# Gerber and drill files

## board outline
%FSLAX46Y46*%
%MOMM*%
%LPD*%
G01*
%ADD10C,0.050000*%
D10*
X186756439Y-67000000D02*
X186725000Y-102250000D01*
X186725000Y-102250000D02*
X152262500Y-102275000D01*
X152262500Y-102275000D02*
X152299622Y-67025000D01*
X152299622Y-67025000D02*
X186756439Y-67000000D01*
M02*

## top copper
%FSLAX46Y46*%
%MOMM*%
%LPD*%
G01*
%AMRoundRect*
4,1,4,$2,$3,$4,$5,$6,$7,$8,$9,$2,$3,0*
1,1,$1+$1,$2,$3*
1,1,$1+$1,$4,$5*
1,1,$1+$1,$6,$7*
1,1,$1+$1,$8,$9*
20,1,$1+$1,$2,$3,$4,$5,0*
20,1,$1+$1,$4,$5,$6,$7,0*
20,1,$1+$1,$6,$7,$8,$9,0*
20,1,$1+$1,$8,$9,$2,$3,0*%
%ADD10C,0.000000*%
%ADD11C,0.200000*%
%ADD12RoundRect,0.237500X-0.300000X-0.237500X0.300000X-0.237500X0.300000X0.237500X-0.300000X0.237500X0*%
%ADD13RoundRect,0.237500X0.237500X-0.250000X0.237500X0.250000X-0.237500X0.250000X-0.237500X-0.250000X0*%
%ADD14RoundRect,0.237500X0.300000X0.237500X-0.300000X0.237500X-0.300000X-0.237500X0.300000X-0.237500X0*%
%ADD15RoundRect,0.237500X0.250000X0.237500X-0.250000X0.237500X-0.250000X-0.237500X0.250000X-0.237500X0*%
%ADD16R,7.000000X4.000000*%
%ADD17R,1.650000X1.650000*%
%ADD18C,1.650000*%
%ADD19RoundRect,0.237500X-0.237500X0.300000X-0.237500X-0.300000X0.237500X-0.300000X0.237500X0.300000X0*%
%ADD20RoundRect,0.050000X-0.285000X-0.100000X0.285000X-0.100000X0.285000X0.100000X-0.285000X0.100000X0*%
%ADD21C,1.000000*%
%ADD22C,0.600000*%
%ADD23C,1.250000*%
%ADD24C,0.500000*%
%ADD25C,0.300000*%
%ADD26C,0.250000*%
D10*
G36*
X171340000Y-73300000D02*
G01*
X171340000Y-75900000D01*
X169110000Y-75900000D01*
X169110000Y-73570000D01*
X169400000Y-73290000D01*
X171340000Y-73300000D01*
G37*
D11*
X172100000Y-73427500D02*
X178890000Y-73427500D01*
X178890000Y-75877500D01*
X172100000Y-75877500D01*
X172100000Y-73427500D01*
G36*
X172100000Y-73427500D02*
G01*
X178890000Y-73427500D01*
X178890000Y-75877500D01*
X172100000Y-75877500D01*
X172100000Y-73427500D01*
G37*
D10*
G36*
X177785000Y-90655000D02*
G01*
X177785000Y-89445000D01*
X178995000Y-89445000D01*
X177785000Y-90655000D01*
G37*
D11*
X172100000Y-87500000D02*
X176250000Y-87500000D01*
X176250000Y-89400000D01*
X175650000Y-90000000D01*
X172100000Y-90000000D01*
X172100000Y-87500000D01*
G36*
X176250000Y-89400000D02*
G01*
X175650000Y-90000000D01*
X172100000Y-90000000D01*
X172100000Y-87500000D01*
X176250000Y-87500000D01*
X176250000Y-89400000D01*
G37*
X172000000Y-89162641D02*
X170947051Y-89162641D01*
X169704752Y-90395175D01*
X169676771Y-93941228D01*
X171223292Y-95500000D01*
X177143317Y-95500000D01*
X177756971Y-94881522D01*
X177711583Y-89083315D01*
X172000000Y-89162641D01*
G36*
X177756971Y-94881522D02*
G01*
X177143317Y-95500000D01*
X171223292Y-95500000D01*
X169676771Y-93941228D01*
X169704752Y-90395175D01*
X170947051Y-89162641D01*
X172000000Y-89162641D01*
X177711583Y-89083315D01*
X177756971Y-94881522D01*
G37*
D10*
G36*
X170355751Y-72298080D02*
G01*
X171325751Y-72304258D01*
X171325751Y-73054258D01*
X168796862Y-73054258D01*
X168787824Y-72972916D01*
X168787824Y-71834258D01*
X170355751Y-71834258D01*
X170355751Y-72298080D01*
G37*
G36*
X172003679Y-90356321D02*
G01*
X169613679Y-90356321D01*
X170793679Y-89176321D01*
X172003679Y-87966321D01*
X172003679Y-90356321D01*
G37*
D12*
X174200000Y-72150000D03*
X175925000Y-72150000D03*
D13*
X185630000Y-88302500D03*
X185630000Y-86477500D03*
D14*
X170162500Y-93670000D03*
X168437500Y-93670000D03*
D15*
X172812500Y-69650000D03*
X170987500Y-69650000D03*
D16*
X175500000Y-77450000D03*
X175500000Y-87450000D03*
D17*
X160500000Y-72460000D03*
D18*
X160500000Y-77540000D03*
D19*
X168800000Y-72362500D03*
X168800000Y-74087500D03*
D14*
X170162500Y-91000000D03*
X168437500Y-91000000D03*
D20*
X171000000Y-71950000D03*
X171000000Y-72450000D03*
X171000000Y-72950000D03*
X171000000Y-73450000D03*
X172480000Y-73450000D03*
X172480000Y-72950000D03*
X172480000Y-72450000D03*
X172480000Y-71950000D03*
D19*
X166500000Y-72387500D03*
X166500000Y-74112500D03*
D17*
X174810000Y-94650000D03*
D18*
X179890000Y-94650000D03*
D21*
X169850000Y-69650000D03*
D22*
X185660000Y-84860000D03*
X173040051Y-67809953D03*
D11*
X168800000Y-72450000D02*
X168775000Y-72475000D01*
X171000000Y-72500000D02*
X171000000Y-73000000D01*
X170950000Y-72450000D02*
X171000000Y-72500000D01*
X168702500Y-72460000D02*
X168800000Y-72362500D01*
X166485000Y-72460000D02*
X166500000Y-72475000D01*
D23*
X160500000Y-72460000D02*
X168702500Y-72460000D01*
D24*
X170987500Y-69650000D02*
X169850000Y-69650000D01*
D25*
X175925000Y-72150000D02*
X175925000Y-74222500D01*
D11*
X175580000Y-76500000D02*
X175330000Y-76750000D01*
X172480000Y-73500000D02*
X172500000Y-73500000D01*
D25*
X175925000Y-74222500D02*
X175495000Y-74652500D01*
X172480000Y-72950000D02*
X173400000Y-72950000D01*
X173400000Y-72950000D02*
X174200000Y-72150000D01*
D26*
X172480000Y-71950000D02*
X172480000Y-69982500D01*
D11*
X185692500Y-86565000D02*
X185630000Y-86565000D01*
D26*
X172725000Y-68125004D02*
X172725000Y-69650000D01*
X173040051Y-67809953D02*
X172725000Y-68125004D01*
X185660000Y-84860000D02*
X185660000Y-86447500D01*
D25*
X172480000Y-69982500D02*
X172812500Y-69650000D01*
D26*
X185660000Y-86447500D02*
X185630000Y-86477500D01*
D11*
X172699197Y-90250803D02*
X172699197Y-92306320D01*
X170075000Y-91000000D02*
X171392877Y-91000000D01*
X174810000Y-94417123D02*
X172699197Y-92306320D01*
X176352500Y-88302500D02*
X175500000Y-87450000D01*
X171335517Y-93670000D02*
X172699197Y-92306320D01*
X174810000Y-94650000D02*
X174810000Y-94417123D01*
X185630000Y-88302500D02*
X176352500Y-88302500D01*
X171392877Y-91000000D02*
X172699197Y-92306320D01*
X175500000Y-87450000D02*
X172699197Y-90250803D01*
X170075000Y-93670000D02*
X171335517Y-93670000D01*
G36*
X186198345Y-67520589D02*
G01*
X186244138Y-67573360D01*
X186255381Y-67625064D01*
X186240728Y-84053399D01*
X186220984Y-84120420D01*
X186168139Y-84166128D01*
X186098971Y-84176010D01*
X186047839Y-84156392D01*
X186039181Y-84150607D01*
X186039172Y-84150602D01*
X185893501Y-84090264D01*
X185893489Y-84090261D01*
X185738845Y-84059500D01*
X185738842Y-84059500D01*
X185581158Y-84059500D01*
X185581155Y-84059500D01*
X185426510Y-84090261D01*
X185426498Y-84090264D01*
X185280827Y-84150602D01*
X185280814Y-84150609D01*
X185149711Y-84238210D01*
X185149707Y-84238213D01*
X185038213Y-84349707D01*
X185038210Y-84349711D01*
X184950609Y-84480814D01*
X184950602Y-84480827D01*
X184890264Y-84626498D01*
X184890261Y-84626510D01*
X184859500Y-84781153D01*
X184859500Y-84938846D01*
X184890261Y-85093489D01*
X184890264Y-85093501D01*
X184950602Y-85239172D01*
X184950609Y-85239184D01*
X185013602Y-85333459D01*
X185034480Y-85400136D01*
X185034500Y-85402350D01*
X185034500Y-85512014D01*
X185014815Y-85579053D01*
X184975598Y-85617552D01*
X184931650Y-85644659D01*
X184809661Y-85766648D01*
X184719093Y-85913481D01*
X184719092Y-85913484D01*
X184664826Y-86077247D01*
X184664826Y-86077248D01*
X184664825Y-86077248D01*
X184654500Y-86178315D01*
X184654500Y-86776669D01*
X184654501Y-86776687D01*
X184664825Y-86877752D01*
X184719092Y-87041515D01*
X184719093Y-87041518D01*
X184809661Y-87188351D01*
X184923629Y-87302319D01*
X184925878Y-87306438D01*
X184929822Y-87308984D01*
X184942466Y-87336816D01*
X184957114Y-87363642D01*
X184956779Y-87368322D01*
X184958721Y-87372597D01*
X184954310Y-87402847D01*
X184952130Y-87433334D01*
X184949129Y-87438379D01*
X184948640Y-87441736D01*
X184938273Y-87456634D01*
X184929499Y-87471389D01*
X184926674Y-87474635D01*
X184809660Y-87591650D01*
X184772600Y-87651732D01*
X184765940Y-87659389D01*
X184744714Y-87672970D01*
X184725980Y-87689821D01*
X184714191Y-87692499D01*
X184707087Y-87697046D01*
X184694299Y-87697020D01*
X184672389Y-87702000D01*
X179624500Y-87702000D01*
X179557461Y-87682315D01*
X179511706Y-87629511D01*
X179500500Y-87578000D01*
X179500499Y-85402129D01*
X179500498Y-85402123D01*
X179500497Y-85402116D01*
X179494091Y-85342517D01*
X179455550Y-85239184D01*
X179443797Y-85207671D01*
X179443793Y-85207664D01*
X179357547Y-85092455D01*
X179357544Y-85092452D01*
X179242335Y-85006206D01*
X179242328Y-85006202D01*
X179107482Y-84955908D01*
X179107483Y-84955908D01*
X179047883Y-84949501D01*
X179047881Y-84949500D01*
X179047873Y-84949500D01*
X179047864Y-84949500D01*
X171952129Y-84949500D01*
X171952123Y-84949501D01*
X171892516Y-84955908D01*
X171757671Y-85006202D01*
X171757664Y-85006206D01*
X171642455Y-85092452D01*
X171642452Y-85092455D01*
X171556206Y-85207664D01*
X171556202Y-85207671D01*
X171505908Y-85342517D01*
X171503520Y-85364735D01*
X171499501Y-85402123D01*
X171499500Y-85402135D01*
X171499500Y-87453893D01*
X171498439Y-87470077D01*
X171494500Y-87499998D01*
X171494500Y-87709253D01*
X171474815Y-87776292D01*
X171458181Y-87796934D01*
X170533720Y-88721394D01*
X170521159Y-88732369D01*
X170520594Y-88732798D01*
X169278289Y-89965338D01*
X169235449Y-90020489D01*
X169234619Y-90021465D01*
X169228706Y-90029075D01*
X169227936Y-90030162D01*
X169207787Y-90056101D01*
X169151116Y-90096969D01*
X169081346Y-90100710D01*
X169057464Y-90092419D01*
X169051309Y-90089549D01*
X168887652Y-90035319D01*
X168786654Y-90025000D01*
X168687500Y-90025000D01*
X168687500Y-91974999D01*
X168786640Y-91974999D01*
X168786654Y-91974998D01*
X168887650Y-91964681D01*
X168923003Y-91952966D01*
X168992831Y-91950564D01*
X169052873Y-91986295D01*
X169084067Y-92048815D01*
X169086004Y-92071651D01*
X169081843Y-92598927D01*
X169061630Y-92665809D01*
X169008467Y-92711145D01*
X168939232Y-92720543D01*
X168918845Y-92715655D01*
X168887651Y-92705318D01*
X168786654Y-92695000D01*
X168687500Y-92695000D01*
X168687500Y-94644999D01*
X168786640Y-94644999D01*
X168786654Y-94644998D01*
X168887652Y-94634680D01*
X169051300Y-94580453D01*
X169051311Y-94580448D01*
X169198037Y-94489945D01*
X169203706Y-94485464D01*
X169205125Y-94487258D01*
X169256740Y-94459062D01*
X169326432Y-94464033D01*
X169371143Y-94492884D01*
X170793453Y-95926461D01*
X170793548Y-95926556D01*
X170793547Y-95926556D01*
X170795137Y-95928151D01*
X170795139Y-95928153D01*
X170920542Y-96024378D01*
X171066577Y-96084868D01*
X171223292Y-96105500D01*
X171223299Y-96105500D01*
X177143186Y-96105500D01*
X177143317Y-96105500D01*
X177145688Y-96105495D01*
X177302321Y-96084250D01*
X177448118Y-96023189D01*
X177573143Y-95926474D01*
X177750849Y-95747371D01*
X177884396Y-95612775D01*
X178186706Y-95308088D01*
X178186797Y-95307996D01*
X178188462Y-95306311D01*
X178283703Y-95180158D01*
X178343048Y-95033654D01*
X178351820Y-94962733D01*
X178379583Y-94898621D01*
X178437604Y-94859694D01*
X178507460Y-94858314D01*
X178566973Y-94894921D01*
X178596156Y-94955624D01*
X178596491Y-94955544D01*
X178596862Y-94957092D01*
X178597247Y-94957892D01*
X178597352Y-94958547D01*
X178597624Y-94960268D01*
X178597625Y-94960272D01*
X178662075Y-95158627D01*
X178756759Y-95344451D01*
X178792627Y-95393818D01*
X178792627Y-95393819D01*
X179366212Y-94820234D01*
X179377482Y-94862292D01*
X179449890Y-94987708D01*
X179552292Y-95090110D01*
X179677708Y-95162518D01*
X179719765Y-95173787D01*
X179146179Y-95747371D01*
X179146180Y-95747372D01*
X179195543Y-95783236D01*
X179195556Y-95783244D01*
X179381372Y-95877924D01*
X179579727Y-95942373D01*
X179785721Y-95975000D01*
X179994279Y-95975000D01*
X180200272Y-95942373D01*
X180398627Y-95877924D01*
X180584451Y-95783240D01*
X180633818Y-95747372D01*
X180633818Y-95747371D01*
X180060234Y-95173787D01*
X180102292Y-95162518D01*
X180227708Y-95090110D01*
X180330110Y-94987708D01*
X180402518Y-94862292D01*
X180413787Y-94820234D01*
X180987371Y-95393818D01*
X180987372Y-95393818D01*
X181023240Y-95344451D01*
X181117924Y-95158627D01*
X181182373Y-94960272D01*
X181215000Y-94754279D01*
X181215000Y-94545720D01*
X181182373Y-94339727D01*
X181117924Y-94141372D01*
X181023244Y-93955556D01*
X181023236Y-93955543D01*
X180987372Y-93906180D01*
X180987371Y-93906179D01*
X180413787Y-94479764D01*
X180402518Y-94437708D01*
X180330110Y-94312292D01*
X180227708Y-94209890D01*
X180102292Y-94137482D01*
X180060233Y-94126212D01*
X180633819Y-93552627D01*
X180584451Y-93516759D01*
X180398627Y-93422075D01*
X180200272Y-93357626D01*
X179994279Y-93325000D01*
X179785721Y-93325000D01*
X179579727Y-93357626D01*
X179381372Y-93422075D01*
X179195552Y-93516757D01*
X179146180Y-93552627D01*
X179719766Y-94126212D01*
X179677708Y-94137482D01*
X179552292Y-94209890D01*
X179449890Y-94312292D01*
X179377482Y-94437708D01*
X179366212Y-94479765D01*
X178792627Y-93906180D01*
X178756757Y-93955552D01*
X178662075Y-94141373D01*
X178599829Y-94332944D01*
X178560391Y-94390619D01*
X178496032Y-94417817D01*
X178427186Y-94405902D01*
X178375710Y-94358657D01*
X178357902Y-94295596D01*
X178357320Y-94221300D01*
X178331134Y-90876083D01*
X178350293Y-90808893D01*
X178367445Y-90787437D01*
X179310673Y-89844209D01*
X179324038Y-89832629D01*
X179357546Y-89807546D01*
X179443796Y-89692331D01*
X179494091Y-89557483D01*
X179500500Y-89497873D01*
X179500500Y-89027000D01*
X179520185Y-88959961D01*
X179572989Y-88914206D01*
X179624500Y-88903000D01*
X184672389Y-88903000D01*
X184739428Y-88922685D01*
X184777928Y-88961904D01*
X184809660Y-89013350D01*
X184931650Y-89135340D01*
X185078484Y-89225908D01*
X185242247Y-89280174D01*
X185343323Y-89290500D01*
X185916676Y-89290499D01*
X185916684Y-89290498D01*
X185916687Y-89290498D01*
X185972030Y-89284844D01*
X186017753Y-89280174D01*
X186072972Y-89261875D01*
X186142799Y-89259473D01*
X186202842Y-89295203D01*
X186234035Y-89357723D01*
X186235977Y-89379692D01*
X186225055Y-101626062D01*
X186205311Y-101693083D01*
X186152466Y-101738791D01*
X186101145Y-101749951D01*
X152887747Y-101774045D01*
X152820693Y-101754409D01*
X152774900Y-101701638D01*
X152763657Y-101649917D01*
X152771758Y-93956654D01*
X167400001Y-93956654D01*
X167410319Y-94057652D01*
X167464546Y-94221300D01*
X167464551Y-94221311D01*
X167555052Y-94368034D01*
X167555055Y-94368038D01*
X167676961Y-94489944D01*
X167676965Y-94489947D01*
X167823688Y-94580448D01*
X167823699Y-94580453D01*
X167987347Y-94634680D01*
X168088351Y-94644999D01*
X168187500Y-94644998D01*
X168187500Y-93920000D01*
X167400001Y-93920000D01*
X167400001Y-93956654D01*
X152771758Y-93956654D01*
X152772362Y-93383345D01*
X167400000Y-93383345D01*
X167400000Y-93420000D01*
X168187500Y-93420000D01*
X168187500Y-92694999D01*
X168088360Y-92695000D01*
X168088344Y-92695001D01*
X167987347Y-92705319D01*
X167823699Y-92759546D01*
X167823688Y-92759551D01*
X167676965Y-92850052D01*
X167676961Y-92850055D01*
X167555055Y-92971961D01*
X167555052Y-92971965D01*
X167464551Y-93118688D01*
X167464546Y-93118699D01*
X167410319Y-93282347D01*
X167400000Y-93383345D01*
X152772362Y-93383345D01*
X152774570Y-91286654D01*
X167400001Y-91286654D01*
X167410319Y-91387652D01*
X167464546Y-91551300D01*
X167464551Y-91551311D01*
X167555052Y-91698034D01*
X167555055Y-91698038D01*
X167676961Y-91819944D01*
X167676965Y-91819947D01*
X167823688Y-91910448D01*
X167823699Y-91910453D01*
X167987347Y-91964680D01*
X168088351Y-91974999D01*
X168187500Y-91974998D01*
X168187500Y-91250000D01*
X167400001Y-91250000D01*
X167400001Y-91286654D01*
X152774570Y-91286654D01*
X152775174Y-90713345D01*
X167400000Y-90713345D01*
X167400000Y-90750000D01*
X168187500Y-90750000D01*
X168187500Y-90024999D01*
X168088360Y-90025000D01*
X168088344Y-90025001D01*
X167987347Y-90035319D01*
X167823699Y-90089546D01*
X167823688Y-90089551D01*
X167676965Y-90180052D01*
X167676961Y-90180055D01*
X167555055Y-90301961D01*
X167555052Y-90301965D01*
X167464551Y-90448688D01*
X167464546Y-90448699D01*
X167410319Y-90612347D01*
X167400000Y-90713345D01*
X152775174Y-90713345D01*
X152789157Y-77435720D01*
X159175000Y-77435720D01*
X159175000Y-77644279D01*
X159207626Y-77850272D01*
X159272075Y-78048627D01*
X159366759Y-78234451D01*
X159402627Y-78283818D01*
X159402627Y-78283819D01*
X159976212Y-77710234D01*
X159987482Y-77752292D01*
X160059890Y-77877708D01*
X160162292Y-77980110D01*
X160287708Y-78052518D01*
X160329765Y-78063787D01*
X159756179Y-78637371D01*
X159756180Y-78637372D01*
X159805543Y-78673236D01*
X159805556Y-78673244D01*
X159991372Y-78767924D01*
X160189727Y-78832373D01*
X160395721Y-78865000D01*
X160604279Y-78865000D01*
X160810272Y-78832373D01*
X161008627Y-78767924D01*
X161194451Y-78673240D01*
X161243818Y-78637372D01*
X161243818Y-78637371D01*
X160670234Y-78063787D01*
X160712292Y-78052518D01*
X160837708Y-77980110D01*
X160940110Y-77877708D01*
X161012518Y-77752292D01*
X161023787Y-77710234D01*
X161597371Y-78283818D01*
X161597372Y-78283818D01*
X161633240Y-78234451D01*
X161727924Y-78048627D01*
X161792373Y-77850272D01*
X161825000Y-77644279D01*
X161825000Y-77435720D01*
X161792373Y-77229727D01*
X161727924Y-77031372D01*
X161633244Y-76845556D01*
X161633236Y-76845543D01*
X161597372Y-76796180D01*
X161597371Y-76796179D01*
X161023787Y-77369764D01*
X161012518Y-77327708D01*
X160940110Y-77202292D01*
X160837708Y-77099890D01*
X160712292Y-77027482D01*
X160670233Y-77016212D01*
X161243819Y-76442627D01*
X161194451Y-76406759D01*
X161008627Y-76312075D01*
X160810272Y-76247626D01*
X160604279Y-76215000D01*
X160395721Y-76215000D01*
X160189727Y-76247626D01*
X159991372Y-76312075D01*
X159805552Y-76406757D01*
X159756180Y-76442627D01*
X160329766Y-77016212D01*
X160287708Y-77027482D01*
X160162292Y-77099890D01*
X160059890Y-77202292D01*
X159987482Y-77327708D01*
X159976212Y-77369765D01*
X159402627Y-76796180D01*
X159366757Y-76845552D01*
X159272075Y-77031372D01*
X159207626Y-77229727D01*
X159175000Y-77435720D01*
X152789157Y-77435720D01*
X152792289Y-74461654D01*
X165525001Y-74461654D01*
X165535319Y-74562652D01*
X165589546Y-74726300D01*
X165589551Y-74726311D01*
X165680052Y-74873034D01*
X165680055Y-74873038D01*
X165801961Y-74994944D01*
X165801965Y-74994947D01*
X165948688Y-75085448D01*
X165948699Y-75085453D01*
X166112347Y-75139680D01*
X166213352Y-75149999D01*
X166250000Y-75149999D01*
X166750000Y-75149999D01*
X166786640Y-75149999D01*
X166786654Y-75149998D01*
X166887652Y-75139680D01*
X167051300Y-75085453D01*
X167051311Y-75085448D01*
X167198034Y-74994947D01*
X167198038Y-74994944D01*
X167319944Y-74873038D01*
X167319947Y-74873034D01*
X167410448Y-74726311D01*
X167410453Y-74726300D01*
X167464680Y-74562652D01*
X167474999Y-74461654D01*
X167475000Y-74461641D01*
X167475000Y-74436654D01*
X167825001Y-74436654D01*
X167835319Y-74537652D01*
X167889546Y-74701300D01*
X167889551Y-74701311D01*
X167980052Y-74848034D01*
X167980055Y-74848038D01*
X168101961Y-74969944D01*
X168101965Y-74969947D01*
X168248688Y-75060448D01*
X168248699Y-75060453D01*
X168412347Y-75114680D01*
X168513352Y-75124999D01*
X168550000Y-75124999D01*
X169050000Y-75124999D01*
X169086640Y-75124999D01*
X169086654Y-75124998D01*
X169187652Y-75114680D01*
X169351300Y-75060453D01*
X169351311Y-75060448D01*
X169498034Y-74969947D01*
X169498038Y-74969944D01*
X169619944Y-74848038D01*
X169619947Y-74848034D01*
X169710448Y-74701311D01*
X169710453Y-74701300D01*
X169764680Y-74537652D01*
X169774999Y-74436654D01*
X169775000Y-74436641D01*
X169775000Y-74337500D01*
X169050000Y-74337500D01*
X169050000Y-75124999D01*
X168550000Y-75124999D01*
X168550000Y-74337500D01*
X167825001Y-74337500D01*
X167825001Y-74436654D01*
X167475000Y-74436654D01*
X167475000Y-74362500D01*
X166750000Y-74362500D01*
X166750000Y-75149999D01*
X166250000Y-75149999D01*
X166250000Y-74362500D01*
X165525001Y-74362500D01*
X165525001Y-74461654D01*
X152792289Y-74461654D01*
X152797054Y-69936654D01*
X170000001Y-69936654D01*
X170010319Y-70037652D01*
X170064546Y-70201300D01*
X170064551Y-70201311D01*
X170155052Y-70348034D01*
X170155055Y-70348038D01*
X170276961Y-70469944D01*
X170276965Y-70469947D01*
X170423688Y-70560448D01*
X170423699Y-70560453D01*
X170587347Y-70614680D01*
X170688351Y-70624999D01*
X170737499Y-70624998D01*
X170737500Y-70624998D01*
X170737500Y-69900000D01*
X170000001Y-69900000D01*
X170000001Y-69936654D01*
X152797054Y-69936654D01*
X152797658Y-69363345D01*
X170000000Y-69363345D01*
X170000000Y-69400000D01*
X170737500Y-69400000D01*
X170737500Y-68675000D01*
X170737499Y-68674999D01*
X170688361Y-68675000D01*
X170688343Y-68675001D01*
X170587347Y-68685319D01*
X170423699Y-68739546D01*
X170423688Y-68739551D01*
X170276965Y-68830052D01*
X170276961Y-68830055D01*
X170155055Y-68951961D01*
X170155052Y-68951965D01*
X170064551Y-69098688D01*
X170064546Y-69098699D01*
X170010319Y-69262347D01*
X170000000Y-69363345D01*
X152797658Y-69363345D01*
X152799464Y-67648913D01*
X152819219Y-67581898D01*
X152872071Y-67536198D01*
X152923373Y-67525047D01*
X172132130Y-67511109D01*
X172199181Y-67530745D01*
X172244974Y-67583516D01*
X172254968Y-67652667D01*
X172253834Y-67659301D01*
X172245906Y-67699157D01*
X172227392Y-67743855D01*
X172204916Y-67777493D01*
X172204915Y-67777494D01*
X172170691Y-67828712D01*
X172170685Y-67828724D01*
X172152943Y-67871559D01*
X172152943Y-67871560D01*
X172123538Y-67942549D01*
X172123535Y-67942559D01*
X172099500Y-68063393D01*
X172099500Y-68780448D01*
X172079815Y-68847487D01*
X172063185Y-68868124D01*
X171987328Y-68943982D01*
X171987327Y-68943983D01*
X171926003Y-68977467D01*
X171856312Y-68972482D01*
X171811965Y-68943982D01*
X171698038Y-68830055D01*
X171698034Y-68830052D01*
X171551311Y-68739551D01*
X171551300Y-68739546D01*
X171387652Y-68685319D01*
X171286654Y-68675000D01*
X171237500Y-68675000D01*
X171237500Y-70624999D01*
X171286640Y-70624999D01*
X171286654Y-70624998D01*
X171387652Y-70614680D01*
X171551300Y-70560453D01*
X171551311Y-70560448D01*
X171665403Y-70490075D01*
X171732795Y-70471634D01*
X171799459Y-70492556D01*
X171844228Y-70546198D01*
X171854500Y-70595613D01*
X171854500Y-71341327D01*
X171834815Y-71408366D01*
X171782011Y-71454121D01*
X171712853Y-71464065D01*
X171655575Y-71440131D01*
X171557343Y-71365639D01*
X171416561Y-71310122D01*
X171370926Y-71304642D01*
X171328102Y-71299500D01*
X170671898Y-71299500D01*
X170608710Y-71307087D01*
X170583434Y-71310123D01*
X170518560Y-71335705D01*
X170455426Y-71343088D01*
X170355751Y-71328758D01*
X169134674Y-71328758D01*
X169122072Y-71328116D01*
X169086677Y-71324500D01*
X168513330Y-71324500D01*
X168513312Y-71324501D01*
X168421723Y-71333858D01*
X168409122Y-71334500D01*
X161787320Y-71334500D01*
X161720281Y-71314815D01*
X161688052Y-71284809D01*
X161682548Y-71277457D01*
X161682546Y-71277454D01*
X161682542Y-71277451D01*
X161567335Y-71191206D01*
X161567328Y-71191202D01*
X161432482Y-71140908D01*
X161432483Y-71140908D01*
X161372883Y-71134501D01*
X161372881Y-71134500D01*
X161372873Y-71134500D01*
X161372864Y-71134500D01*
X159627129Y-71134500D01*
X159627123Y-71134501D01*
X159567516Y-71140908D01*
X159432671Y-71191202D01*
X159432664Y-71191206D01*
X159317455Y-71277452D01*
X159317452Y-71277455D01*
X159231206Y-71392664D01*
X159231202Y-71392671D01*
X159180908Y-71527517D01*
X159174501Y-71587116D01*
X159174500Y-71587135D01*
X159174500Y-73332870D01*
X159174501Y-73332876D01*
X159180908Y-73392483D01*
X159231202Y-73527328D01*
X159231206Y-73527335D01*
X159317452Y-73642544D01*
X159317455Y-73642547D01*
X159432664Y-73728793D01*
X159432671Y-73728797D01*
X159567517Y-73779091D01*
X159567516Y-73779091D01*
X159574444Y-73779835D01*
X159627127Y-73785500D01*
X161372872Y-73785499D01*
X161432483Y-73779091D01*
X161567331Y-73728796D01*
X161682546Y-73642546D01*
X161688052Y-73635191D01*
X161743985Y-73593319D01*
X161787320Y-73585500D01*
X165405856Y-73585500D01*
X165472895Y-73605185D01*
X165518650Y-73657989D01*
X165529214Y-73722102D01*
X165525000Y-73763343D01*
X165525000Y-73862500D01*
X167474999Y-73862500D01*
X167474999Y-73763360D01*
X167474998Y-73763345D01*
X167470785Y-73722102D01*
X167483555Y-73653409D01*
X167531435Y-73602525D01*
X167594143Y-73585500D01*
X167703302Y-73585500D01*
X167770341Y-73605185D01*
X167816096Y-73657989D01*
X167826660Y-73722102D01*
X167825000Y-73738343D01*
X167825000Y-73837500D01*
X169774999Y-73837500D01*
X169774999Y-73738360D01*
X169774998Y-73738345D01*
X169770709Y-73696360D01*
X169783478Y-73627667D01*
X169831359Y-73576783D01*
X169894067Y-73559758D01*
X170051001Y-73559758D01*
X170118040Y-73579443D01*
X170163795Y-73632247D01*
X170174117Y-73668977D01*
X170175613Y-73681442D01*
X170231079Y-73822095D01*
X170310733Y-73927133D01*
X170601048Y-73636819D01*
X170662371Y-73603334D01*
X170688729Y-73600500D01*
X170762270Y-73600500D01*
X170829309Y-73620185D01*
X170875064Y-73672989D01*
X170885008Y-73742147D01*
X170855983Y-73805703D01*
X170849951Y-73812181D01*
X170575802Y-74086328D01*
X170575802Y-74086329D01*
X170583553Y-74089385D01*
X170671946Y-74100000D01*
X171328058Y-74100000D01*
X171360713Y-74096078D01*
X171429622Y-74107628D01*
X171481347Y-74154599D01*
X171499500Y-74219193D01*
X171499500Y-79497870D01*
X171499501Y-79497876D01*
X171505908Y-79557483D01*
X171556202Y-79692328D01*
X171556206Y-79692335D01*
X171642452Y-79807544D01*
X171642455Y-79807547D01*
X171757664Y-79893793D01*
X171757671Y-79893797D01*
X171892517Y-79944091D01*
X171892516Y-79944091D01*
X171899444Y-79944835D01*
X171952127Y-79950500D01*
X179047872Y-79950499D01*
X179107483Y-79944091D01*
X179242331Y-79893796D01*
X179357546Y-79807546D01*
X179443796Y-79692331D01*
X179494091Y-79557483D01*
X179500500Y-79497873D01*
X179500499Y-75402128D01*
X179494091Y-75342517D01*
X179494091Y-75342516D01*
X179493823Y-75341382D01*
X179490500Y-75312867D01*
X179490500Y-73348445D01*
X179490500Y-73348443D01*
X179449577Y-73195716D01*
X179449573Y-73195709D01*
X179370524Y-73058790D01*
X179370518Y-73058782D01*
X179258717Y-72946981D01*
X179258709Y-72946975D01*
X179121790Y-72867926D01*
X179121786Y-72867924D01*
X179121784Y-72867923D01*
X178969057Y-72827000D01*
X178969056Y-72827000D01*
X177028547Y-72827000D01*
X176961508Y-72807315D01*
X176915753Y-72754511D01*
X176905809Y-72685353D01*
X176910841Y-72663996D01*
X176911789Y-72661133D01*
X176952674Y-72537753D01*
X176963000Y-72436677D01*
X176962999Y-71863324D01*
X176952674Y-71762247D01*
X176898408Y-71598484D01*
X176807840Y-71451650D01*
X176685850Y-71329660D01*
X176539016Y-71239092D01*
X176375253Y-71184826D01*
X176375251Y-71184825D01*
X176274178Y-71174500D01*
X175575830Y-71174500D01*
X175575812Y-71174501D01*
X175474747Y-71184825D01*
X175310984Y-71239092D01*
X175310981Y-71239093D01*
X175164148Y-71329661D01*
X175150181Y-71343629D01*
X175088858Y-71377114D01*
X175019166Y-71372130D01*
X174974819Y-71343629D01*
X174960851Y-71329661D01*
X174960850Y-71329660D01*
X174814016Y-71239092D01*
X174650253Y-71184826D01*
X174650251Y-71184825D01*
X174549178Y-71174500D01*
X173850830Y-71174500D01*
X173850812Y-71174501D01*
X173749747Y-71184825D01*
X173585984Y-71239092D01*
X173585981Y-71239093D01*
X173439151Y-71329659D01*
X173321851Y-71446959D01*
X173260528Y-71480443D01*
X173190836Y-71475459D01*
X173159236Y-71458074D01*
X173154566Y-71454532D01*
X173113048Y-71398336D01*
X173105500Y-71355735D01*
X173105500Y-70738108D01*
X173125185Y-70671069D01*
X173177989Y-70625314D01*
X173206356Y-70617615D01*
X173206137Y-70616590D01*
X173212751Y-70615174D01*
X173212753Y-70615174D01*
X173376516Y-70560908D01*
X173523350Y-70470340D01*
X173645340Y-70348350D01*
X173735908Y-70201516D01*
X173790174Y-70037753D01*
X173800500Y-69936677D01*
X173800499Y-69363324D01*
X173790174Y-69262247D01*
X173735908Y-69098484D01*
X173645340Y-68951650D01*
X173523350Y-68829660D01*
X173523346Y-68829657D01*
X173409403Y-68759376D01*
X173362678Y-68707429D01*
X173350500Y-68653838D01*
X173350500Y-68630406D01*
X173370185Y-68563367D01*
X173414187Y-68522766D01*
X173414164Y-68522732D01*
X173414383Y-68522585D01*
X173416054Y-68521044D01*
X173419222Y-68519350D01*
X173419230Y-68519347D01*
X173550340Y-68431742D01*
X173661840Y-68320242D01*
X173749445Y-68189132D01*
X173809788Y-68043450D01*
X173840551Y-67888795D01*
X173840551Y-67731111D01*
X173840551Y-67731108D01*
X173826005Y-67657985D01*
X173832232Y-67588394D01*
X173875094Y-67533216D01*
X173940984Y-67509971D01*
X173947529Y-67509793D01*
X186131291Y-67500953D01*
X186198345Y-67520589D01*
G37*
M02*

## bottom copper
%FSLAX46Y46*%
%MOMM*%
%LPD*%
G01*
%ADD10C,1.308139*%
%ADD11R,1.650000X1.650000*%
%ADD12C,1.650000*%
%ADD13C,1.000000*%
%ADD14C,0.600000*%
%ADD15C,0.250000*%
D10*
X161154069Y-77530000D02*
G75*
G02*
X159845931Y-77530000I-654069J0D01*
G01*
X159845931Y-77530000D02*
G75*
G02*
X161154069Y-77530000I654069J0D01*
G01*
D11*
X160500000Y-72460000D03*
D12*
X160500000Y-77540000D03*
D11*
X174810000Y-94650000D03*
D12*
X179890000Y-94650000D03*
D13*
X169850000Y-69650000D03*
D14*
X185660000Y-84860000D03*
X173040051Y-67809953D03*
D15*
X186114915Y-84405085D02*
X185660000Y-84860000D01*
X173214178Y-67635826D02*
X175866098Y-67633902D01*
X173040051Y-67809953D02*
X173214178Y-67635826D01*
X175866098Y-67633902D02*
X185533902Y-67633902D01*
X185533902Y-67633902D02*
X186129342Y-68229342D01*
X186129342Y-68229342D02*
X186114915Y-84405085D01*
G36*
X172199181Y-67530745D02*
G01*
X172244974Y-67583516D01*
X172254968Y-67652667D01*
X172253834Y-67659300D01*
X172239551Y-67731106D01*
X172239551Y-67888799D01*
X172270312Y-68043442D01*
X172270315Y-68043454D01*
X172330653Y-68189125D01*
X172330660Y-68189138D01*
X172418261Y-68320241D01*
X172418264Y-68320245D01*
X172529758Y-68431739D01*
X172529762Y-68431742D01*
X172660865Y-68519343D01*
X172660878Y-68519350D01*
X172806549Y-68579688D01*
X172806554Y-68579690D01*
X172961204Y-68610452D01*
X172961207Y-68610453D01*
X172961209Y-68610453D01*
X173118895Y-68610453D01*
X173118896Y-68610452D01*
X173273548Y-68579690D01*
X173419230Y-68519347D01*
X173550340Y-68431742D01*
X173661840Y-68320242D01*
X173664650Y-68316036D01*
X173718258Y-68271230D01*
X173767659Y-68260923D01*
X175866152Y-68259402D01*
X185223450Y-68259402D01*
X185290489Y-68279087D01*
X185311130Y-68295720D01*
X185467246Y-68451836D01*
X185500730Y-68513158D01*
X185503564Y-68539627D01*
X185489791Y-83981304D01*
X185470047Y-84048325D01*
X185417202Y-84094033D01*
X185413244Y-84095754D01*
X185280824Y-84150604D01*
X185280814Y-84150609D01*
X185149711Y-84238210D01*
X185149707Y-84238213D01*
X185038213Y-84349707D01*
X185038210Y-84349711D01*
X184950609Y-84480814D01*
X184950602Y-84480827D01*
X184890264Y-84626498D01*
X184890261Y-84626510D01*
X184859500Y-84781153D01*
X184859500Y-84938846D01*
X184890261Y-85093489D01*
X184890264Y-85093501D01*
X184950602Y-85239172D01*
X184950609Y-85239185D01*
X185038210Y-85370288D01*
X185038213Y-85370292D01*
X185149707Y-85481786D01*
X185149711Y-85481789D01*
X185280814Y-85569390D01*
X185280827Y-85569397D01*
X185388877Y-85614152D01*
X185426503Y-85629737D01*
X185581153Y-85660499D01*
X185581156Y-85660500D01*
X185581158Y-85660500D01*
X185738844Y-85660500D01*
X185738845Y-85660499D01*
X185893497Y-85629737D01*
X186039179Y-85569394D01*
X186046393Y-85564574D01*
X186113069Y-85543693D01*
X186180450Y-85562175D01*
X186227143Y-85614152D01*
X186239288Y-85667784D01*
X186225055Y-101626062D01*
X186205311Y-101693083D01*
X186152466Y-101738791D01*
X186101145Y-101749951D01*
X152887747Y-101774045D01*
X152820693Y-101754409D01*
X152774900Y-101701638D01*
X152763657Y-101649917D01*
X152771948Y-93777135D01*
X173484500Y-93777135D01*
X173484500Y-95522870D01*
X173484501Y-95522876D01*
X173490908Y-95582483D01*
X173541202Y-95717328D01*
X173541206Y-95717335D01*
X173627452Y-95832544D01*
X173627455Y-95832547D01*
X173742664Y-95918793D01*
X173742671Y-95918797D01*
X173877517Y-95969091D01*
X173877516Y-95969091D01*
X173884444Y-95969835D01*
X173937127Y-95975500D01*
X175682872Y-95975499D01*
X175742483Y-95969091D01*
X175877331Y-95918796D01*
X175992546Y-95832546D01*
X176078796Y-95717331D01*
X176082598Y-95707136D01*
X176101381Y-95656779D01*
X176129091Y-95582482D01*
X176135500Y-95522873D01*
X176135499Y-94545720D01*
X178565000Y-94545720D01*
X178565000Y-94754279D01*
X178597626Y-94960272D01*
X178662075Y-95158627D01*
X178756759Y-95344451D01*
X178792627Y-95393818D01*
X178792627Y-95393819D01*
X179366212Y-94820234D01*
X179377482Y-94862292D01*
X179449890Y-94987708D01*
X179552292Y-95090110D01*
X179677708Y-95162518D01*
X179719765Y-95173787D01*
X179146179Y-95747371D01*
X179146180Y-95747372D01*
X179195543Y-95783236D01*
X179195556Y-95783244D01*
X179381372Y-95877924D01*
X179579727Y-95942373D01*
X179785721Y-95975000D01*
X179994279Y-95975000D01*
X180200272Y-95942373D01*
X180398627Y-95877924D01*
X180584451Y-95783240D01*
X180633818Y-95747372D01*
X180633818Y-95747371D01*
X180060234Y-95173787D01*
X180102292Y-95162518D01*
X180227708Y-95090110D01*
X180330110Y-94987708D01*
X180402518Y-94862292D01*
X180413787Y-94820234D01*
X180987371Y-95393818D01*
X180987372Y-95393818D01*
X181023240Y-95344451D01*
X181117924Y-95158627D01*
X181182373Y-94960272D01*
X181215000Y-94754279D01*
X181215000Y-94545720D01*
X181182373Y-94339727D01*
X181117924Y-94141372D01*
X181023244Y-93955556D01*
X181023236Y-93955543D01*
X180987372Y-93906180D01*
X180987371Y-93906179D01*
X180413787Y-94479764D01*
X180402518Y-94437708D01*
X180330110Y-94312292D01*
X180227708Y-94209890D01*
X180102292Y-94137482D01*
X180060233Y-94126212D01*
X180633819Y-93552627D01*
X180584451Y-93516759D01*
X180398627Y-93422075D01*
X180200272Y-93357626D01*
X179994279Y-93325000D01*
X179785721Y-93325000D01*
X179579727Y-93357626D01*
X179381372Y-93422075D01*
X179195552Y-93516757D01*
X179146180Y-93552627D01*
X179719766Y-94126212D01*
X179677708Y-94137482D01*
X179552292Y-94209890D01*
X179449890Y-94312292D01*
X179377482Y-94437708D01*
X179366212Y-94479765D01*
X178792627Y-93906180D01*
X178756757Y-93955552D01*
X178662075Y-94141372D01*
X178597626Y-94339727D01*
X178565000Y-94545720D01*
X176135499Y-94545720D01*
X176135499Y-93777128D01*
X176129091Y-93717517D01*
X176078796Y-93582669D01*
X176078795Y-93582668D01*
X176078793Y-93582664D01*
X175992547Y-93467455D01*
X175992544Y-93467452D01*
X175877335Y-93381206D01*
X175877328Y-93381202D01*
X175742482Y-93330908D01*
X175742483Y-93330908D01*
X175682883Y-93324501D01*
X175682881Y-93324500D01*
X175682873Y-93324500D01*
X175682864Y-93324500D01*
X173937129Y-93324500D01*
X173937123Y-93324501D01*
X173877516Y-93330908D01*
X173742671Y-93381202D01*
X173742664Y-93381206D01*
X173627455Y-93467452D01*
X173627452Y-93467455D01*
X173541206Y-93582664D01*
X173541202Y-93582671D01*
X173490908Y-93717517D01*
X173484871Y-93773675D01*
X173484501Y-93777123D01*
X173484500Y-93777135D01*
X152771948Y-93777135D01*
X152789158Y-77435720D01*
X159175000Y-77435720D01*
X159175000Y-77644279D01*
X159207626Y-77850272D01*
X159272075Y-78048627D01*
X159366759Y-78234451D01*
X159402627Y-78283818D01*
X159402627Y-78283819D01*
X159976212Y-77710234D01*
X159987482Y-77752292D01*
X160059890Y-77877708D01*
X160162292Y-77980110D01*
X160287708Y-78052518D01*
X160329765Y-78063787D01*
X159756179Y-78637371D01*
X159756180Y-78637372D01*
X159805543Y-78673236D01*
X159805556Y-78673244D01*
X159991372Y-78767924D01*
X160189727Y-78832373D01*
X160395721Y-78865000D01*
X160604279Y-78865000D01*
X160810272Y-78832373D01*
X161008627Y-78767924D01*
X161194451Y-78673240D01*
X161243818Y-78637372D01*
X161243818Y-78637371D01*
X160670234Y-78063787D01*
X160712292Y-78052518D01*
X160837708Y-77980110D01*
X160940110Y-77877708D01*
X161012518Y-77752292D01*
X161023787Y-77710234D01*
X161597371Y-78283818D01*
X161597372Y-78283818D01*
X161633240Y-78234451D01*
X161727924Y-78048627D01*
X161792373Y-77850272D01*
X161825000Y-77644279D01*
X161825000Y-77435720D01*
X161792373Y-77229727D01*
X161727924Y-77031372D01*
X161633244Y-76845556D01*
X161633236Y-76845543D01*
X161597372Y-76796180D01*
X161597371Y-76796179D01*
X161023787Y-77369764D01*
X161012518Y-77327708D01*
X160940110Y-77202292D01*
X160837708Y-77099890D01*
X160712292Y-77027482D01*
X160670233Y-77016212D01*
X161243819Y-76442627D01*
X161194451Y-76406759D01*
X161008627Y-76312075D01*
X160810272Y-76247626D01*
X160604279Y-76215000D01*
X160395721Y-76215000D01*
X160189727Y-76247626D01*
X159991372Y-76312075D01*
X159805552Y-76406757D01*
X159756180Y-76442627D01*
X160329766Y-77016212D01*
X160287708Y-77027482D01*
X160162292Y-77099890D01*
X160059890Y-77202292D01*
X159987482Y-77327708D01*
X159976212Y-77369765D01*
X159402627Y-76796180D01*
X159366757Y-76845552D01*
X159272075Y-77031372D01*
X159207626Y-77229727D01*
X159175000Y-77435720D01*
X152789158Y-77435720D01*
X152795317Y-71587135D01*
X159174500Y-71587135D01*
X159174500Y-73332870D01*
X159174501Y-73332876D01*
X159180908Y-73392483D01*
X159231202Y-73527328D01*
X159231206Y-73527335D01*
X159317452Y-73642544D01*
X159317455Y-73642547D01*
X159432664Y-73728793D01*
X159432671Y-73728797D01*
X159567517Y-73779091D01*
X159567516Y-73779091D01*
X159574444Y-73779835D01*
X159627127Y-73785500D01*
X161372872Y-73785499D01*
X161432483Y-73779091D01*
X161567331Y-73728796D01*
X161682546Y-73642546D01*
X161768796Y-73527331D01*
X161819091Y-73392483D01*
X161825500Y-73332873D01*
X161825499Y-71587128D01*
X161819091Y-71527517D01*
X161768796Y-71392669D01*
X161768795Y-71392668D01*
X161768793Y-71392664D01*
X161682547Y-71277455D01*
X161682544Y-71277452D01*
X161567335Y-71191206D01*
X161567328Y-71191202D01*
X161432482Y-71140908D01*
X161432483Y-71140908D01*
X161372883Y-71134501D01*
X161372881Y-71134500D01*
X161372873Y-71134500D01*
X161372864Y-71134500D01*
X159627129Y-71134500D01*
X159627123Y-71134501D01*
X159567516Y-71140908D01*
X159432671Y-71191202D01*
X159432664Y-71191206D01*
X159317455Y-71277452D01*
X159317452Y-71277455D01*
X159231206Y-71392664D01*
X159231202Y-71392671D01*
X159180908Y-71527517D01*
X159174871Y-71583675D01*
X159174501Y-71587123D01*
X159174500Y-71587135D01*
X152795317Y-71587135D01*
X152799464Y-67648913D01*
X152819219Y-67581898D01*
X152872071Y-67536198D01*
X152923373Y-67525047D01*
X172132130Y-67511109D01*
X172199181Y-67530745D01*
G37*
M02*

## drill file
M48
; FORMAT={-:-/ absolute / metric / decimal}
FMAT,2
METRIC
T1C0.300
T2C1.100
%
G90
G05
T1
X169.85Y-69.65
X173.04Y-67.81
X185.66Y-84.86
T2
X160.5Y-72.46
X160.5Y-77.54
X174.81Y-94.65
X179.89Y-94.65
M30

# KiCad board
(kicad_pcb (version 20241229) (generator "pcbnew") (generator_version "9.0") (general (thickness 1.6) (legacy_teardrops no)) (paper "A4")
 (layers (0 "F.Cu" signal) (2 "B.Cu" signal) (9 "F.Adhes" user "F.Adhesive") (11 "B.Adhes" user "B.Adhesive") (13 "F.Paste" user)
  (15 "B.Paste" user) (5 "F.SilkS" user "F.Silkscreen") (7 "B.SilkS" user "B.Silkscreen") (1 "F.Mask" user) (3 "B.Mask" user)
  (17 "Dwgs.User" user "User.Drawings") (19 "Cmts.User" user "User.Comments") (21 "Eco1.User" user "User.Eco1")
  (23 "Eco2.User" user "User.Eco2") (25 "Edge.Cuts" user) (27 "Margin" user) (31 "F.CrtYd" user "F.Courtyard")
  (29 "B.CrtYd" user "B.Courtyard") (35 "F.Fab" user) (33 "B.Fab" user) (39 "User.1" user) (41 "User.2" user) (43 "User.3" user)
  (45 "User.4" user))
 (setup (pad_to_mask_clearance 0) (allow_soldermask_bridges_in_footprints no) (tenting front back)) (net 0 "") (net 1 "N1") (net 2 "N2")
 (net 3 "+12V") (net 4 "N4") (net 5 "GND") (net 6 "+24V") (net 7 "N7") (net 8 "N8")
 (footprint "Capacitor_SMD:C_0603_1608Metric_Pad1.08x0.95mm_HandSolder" (layer "F.Cu") (at 175.0625 72.15)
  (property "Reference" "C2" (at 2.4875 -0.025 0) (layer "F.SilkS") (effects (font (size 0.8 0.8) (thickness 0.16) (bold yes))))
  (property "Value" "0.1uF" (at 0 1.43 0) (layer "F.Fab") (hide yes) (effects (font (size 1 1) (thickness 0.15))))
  (pad "1" smd roundrect (at -0.8625 0) (size 1.075 0.95) (layers "F.Cu" "F.Mask" "F.Paste") (roundrect_rratio 0.25) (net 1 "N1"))
  (pad "2" smd roundrect (at 0.8625 0) (size 1.075 0.95) (layers "F.Cu" "F.Mask" "F.Paste") (roundrect_rratio 0.25) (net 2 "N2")))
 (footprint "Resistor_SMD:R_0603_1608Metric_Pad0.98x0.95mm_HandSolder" (layer "F.Cu") (at 185.63 87.39 90)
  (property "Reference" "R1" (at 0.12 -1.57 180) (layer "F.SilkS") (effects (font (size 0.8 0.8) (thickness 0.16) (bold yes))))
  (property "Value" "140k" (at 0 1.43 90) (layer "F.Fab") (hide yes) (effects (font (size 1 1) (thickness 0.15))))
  (pad "1" smd roundrect (at -0.9125 0 90) (size 0.975 0.95) (layers "F.Cu" "F.Mask" "F.Paste") (roundrect_rratio 0.25) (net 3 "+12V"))
  (pad "2" smd roundrect (at 0.9125 0 90) (size 0.975 0.95) (layers "F.Cu" "F.Mask" "F.Paste") (roundrect_rratio 0.25) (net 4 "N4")))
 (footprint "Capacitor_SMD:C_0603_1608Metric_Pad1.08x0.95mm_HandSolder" (layer "F.Cu") (at 169.3 93.67 180)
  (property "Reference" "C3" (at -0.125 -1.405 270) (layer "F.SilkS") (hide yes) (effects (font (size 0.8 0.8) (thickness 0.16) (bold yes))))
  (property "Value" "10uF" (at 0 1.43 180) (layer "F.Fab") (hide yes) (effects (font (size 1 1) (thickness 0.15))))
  (pad "1" smd roundrect (at -0.8625 0 180) (size 1.075 0.95) (layers "F.Cu" "F.Mask" "F.Paste") (roundrect_rratio 0.25) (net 3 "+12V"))
  (pad "2" smd roundrect (at 0.8625 0 180) (size 1.075 0.95) (layers "F.Cu" "F.Mask" "F.Paste") (roundrect_rratio 0.25) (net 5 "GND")))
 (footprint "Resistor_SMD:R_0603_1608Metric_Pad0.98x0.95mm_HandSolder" (layer "F.Cu") (at 171.9 69.65 180)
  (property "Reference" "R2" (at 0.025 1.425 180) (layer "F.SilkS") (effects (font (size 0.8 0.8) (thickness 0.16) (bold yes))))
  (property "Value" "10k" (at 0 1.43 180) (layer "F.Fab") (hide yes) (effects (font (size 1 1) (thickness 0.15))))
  (pad "1" smd roundrect (at -0.9125 0 180) (size 0.975 0.95) (layers "F.Cu" "F.Mask" "F.Paste") (roundrect_rratio 0.25) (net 4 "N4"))
  (pad "2" smd roundrect (at 0.9125 0 180) (size 0.975 0.95) (layers "F.Cu" "F.Mask" "F.Paste") (roundrect_rratio 0.25) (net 5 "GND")))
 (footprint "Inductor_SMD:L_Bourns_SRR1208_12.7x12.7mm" (layer "F.Cu") (at 175.5 82.45 -90)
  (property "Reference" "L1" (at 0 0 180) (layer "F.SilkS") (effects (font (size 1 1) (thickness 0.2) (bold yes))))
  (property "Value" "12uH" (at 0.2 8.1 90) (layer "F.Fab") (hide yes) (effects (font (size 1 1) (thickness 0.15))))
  (pad "1" smd rect (at -5 0 270) (size 4 7) (layers "F.Cu" "F.Mask" "F.Paste") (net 2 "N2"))
  (pad "2" smd rect (at 5 0 270) (size 4 7) (layers "F.Cu" "F.Mask" "F.Paste") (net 3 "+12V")))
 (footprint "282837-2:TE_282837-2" (layer "F.Cu") (at 160.5 75 -90)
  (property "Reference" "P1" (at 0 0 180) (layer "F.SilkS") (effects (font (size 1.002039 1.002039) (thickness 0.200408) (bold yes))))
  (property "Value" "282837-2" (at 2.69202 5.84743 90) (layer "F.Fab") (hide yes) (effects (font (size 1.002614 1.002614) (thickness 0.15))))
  (pad "1" thru_hole rect (at -2.54 0 270) (size 1.65 1.65) (drill 1.1) (layers "*.Cu" "*.Mask") (remove_unused_layers no) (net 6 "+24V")
   (solder_mask_margin 0.102))
  (pad "2" thru_hole circle (at 2.54 0 270) (size 1.65 1.65) (drill 1.1) (layers "*.Cu" "*.Mask") (remove_unused_layers no) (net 5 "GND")
   (solder_mask_margin 0.102)))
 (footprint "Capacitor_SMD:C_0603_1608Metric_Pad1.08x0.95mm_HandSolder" (layer "F.Cu") (at 168.8 73.225 -90)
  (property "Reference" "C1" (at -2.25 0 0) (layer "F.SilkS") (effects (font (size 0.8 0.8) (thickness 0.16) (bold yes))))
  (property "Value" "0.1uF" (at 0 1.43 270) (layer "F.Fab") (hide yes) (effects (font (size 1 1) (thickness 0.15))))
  (pad "1" smd roundrect (at -0.8625 0 270) (size 1.075 0.95) (layers "F.Cu" "F.Mask" "F.Paste") (roundrect_rratio 0.25) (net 6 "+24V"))
  (pad "2" smd roundrect (at 0.8625 0 270) (size 1.075 0.95) (layers "F.Cu" "F.Mask" "F.Paste") (roundrect_rratio 0.25) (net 5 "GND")))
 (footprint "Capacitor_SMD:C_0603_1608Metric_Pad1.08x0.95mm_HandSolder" (layer "F.Cu") (at 169.3 91 180)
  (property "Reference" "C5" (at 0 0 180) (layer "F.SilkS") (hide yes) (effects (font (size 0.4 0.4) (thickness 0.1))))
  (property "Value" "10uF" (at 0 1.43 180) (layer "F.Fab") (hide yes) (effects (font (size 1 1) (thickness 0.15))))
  (pad "1" smd roundrect (at -0.8625 0 180) (size 1.075 0.95) (layers "F.Cu" "F.Mask" "F.Paste") (roundrect_rratio 0.25) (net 3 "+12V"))
  (pad "2" smd roundrect (at 0.8625 0 180) (size 1.075 0.95) (layers "F.Cu" "F.Mask" "F.Paste") (roundrect_rratio 0.25) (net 5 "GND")))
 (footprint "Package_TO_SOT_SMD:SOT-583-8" (layer "F.Cu") (at 171.74 72.7)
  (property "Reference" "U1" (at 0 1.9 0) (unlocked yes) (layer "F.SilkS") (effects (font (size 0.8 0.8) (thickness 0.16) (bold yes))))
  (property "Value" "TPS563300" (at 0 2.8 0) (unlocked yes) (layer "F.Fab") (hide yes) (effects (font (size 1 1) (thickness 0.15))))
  (pad "1" smd roundrect (at -0.74 -0.75) (size 0.67 0.3) (layers "F.Cu" "F.Mask" "F.Paste") (roundrect_rratio 0.1666666667) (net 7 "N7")
   (thermal_bridge_angle 45))
  (pad "2" smd roundrect (at -0.74 -0.25) (size 0.67 0.3) (layers "F.Cu" "F.Mask" "F.Paste") (roundrect_rratio 0.1666666667) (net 6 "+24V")
   (thermal_bridge_angle 45))
  (pad "3" smd roundrect (at -0.74 0.25) (size 0.67 0.3) (layers "F.Cu" "F.Mask" "F.Paste") (roundrect_rratio 0.1666666667) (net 6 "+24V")
   (thermal_bridge_angle 45))
  (pad "4" smd roundrect (at -0.74 0.75) (size 0.67 0.3) (layers "F.Cu" "F.Mask" "F.Paste") (roundrect_rratio 0.1666666667) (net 5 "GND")
   (thermal_bridge_angle 45))
  (pad "5" smd roundrect (at 0.74 0.75) (size 0.67 0.3) (layers "F.Cu" "F.Mask" "F.Paste") (roundrect_rratio 0.1666666667) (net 2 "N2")
   (thermal_bridge_angle 45))
  (pad "6" smd roundrect (at 0.74 0.25) (size 0.67 0.3) (layers "F.Cu" "F.Mask" "F.Paste") (roundrect_rratio 0.1666666667) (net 1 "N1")
   (thermal_bridge_angle 45))
  (pad "7" smd roundrect (at 0.74 -0.25) (size 0.67 0.3) (layers "F.Cu" "F.Mask" "F.Paste") (roundrect_rratio 0.1666666667) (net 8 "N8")
   (thermal_bridge_angle 45))
  (pad "8" smd roundrect (at 0.74 -0.75) (size 0.67 0.3) (layers "F.Cu" "F.Mask" "F.Paste") (roundrect_rratio 0.1666666667) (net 4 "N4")
   (thermal_bridge_angle 45)))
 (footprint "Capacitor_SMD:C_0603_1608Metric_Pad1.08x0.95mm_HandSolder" (layer "F.Cu") (at 166.5 73.25 -90)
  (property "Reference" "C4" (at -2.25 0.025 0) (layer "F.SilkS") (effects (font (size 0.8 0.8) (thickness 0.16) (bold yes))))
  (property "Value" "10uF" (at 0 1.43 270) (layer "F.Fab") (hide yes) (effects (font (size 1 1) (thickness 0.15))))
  (pad "1" smd roundrect (at -0.8625 0 270) (size 1.075 0.95) (layers "F.Cu" "F.Mask" "F.Paste") (roundrect_rratio 0.25) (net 6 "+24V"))
  (pad "2" smd roundrect (at 0.8625 0 270) (size 1.075 0.95) (layers "F.Cu" "F.Mask" "F.Paste") (roundrect_rratio 0.25) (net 5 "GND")))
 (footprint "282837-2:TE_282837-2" (layer "F.Cu") (at 177.35 94.65)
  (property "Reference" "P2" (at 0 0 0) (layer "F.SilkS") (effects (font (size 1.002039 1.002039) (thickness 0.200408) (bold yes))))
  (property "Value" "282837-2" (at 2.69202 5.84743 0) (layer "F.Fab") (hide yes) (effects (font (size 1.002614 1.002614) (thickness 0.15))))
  (pad "1" thru_hole rect (at -2.54 0) (size 1.65 1.65) (drill 1.1) (layers "*.Cu" "*.Mask") (remove_unused_layers no) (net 3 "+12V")
   (solder_mask_margin 0.102))
  (pad "2" thru_hole circle (at 2.54 0) (size 1.65 1.65) (drill 1.1) (layers "*.Cu" "*.Mask") (remove_unused_layers no) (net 5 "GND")
   (solder_mask_margin 0.102)))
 (gr_poly
  (pts (xy 169.11 73.57) (xy 169.4 73.29) (xy 171.34 73.3) (xy 171.34 75.9) (xy 169.11 75.9)) (stroke (width 0) (type solid)) (fill yes)
  (layer "F.Cu") (net 5))
 (gr_rect (start 172.1 73.4275) (end 178.89 75.8775) (stroke (width 0.2) (type solid)) (fill yes) (layer "F.Cu") (net 2))
 (gr_poly
  (pts (xy 178.995 89.445) (xy 177.785 90.655) (xy 177.785 89.445) (xy 178.995 89.445)) (stroke (width 0) (type solid)) (fill yes)
  (layer "F.Cu") (net 3))
 (gr_poly
  (pts (xy 172.1 87.5) (xy 176.25 87.5) (xy 176.25 89.4) (xy 175.65 90) (xy 172.1 90)) (stroke (width 0.2) (type solid)) (fill yes)
  (layer "F.Cu") (net 3))
 (gr_poly
  (pts (xy 172 89.162641) (xy 170.947051 89.162641) (xy 169.704752 90.395175) (xy 169.676771 93.941228) (xy 171.223292 95.5)
   (xy 177.143317 95.5) (xy 177.756971 94.881522) (xy 177.711583 89.083315))
  (stroke (width 0.2) (type solid)) (fill yes) (layer "F.Cu") (net 3))
 (gr_poly
  (pts (xy 168.787824 71.834258) (xy 170.355751 71.834258) (xy 170.355751 72.29808) (xy 171.325751 72.304258) (xy 171.325751 73.054258)
   (xy 168.796862 73.054258) (xy 168.787824 72.972916))
  (stroke (width 0) (type solid)) (fill yes) (layer "F.Cu") (net 6))
 (gr_poly
  (pts (xy 170.793679 89.176321) (xy 172.003679 87.966321) (xy 172.003679 90.356321) (xy 169.613679 90.356321))
  (stroke (width 0) (type solid)) (fill yes) (layer "F.Cu") (net 3))
 (gr_circle (center 160.5 77.53) (end 160.36 76.33) (stroke (width 0.2) (type solid)) (fill yes) (layer "B.Cu") (net 5))
 (gr_line (start 186.756439 67) (end 186.725 102.25) (stroke (width 0.05) (type default)) (layer "Edge.Cuts"))
 (gr_line (start 186.725 102.25) (end 152.2625 102.275) (stroke (width 0.05) (type default)) (layer "Edge.Cuts"))
 (gr_line (start 152.2625 102.275) (end 152.299622 67.025) (stroke (width 0.05) (type default)) (layer "Edge.Cuts"))
 (gr_line (start 152.299622 67.025) (end 186.756439 67) (stroke (width 0.05) (type default)) (layer "Edge.Cuts"))
 (segment (start 168.8 72.45) (end 168.775 72.475) (width 0.2) (layer "F.Cu") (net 6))
 (segment (start 171 72.5) (end 171 73) (width 0.2) (layer "F.Cu") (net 6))
 (segment (start 170.95 72.45) (end 171 72.5) (width 0.2) (layer "F.Cu") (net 6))
 (segment (start 168.7025 72.46) (end 168.8 72.3625) (width 0.2) (layer "F.Cu") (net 6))
 (segment (start 166.485 72.46) (end 166.5 72.475) (width 0.2) (layer "F.Cu") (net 6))
 (segment (start 160.5 72.46) (end 168.7025 72.46) (width 1.25) (layer "F.Cu") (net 6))
 (segment (start 170.9875 69.65) (end 169.85 69.65) (width 0.5) (layer "F.Cu") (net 5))
 (via (at 169.85 69.65) (size 1) (drill 0.3) (layers "F.Cu" "B.Cu") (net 5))
 (segment (start 175.925 72.15) (end 175.925 74.2225) (width 0.3) (layer "F.Cu") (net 2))
 (segment (start 175.58 76.5) (end 175.33 76.75) (width 0.2) (layer "F.Cu") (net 2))
 (segment (start 172.48 73.5) (end 172.5 73.5) (width 0.2) (layer "F.Cu") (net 2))
 (segment (start 175.925 74.2225) (end 175.495 74.6525) (width 0.3) (layer "F.Cu") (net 2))
 (segment (start 172.48 72.95) (end 173.4 72.95) (width 0.3) (layer "F.Cu") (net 1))
 (segment (start 173.4 72.95) (end 174.2 72.15) (width 0.3) (layer "F.Cu") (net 1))
 (segment (start 172.48 71.95) (end 172.48 69.9825) (width 0.25) (layer "F.Cu") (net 4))
 (segment (start 185.6925 86.565) (end 185.63 86.565) (width 0.2) (layer "F.Cu") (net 4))
 (segment (start 172.725 68.125004) (end 172.725 69.65) (width 0.25) (layer "F.Cu") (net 4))
 (segment (start 173.040051 67.809953) (end 172.725 68.125004) (width 0.25) (layer "F.Cu") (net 4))
 (segment (start 185.66 84.86) (end 185.66 86.4475) (width 0.25) (layer "F.Cu") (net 4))
 (segment (start 172.48 69.9825) (end 172.8125 69.65) (width 0.3) (layer "F.Cu") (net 4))
 (segment (start 185.66 86.4475) (end 185.63 86.4775) (width 0.25) (layer "F.Cu") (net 4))
 (via (at 185.66 84.86) (size 0.6) (drill 0.3) (layers "F.Cu" "B.Cu") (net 4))
 (via (at 173.040051 67.809953) (size 0.6) (drill 0.3) (layers "F.Cu" "B.Cu") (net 4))
 (segment (start 186.114915 84.405085) (end 185.66 84.86) (width 0.25) (layer "B.Cu") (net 4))
 (segment (start 173.214178 67.635826) (end 175.866098 67.633902) (width 0.25) (layer "B.Cu") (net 4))
 (segment (start 173.040051 67.809953) (end 173.214178 67.635826) (width 0.25) (layer "B.Cu") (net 4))
 (segment (start 175.866098 67.633902) (end 185.533902 67.633902) (width 0.25) (layer "B.Cu") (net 4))
 (segment (start 185.533902 67.633902) (end 186.129342 68.229342) (width 0.25) (layer "B.Cu") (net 4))
 (segment (start 186.129342 68.229342) (end 186.114915 84.405085) (width 0.25) (layer "B.Cu") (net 4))
 (segment (start 172.699197 90.250803) (end 172.699197 92.30632) (width 0.2) (layer "F.Cu") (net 3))
 (segment (start 170.075 91) (end 171.392877 91) (width 0.2) (layer "F.Cu") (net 3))
 (segment (start 174.81 94.417123) (end 172.699197 92.30632) (width 0.2) (layer "F.Cu") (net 3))
 (segment (start 176.3525 88.3025) (end 175.5 87.45) (width 0.2) (layer "F.Cu") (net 3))
 (segment (start 171.335517 93.67) (end 172.699197 92.30632) (width 0.2) (layer "F.Cu") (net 3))
 (segment (start 174.81 94.65) (end 174.81 94.417123) (width 0.2) (layer "F.Cu") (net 3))
 (segment (start 185.63 88.3025) (end 176.3525 88.3025) (width 0.2) (layer "F.Cu") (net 3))
 (segment (start 171.392877 91) (end 172.699197 92.30632) (width 0.2) (layer "F.Cu") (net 3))
 (segment (start 175.5 87.45) (end 172.699197 90.250803) (width 0.2) (layer "F.Cu") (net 3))
 (segment (start 170.075 93.67) (end 171.335517 93.67) (width 0.2) (layer "F.Cu") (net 3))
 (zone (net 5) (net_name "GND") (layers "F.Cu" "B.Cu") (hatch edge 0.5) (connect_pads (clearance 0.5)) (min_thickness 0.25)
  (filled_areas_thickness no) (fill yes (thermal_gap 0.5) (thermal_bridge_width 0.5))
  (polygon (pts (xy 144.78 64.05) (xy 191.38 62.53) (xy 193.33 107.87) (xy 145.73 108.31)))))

